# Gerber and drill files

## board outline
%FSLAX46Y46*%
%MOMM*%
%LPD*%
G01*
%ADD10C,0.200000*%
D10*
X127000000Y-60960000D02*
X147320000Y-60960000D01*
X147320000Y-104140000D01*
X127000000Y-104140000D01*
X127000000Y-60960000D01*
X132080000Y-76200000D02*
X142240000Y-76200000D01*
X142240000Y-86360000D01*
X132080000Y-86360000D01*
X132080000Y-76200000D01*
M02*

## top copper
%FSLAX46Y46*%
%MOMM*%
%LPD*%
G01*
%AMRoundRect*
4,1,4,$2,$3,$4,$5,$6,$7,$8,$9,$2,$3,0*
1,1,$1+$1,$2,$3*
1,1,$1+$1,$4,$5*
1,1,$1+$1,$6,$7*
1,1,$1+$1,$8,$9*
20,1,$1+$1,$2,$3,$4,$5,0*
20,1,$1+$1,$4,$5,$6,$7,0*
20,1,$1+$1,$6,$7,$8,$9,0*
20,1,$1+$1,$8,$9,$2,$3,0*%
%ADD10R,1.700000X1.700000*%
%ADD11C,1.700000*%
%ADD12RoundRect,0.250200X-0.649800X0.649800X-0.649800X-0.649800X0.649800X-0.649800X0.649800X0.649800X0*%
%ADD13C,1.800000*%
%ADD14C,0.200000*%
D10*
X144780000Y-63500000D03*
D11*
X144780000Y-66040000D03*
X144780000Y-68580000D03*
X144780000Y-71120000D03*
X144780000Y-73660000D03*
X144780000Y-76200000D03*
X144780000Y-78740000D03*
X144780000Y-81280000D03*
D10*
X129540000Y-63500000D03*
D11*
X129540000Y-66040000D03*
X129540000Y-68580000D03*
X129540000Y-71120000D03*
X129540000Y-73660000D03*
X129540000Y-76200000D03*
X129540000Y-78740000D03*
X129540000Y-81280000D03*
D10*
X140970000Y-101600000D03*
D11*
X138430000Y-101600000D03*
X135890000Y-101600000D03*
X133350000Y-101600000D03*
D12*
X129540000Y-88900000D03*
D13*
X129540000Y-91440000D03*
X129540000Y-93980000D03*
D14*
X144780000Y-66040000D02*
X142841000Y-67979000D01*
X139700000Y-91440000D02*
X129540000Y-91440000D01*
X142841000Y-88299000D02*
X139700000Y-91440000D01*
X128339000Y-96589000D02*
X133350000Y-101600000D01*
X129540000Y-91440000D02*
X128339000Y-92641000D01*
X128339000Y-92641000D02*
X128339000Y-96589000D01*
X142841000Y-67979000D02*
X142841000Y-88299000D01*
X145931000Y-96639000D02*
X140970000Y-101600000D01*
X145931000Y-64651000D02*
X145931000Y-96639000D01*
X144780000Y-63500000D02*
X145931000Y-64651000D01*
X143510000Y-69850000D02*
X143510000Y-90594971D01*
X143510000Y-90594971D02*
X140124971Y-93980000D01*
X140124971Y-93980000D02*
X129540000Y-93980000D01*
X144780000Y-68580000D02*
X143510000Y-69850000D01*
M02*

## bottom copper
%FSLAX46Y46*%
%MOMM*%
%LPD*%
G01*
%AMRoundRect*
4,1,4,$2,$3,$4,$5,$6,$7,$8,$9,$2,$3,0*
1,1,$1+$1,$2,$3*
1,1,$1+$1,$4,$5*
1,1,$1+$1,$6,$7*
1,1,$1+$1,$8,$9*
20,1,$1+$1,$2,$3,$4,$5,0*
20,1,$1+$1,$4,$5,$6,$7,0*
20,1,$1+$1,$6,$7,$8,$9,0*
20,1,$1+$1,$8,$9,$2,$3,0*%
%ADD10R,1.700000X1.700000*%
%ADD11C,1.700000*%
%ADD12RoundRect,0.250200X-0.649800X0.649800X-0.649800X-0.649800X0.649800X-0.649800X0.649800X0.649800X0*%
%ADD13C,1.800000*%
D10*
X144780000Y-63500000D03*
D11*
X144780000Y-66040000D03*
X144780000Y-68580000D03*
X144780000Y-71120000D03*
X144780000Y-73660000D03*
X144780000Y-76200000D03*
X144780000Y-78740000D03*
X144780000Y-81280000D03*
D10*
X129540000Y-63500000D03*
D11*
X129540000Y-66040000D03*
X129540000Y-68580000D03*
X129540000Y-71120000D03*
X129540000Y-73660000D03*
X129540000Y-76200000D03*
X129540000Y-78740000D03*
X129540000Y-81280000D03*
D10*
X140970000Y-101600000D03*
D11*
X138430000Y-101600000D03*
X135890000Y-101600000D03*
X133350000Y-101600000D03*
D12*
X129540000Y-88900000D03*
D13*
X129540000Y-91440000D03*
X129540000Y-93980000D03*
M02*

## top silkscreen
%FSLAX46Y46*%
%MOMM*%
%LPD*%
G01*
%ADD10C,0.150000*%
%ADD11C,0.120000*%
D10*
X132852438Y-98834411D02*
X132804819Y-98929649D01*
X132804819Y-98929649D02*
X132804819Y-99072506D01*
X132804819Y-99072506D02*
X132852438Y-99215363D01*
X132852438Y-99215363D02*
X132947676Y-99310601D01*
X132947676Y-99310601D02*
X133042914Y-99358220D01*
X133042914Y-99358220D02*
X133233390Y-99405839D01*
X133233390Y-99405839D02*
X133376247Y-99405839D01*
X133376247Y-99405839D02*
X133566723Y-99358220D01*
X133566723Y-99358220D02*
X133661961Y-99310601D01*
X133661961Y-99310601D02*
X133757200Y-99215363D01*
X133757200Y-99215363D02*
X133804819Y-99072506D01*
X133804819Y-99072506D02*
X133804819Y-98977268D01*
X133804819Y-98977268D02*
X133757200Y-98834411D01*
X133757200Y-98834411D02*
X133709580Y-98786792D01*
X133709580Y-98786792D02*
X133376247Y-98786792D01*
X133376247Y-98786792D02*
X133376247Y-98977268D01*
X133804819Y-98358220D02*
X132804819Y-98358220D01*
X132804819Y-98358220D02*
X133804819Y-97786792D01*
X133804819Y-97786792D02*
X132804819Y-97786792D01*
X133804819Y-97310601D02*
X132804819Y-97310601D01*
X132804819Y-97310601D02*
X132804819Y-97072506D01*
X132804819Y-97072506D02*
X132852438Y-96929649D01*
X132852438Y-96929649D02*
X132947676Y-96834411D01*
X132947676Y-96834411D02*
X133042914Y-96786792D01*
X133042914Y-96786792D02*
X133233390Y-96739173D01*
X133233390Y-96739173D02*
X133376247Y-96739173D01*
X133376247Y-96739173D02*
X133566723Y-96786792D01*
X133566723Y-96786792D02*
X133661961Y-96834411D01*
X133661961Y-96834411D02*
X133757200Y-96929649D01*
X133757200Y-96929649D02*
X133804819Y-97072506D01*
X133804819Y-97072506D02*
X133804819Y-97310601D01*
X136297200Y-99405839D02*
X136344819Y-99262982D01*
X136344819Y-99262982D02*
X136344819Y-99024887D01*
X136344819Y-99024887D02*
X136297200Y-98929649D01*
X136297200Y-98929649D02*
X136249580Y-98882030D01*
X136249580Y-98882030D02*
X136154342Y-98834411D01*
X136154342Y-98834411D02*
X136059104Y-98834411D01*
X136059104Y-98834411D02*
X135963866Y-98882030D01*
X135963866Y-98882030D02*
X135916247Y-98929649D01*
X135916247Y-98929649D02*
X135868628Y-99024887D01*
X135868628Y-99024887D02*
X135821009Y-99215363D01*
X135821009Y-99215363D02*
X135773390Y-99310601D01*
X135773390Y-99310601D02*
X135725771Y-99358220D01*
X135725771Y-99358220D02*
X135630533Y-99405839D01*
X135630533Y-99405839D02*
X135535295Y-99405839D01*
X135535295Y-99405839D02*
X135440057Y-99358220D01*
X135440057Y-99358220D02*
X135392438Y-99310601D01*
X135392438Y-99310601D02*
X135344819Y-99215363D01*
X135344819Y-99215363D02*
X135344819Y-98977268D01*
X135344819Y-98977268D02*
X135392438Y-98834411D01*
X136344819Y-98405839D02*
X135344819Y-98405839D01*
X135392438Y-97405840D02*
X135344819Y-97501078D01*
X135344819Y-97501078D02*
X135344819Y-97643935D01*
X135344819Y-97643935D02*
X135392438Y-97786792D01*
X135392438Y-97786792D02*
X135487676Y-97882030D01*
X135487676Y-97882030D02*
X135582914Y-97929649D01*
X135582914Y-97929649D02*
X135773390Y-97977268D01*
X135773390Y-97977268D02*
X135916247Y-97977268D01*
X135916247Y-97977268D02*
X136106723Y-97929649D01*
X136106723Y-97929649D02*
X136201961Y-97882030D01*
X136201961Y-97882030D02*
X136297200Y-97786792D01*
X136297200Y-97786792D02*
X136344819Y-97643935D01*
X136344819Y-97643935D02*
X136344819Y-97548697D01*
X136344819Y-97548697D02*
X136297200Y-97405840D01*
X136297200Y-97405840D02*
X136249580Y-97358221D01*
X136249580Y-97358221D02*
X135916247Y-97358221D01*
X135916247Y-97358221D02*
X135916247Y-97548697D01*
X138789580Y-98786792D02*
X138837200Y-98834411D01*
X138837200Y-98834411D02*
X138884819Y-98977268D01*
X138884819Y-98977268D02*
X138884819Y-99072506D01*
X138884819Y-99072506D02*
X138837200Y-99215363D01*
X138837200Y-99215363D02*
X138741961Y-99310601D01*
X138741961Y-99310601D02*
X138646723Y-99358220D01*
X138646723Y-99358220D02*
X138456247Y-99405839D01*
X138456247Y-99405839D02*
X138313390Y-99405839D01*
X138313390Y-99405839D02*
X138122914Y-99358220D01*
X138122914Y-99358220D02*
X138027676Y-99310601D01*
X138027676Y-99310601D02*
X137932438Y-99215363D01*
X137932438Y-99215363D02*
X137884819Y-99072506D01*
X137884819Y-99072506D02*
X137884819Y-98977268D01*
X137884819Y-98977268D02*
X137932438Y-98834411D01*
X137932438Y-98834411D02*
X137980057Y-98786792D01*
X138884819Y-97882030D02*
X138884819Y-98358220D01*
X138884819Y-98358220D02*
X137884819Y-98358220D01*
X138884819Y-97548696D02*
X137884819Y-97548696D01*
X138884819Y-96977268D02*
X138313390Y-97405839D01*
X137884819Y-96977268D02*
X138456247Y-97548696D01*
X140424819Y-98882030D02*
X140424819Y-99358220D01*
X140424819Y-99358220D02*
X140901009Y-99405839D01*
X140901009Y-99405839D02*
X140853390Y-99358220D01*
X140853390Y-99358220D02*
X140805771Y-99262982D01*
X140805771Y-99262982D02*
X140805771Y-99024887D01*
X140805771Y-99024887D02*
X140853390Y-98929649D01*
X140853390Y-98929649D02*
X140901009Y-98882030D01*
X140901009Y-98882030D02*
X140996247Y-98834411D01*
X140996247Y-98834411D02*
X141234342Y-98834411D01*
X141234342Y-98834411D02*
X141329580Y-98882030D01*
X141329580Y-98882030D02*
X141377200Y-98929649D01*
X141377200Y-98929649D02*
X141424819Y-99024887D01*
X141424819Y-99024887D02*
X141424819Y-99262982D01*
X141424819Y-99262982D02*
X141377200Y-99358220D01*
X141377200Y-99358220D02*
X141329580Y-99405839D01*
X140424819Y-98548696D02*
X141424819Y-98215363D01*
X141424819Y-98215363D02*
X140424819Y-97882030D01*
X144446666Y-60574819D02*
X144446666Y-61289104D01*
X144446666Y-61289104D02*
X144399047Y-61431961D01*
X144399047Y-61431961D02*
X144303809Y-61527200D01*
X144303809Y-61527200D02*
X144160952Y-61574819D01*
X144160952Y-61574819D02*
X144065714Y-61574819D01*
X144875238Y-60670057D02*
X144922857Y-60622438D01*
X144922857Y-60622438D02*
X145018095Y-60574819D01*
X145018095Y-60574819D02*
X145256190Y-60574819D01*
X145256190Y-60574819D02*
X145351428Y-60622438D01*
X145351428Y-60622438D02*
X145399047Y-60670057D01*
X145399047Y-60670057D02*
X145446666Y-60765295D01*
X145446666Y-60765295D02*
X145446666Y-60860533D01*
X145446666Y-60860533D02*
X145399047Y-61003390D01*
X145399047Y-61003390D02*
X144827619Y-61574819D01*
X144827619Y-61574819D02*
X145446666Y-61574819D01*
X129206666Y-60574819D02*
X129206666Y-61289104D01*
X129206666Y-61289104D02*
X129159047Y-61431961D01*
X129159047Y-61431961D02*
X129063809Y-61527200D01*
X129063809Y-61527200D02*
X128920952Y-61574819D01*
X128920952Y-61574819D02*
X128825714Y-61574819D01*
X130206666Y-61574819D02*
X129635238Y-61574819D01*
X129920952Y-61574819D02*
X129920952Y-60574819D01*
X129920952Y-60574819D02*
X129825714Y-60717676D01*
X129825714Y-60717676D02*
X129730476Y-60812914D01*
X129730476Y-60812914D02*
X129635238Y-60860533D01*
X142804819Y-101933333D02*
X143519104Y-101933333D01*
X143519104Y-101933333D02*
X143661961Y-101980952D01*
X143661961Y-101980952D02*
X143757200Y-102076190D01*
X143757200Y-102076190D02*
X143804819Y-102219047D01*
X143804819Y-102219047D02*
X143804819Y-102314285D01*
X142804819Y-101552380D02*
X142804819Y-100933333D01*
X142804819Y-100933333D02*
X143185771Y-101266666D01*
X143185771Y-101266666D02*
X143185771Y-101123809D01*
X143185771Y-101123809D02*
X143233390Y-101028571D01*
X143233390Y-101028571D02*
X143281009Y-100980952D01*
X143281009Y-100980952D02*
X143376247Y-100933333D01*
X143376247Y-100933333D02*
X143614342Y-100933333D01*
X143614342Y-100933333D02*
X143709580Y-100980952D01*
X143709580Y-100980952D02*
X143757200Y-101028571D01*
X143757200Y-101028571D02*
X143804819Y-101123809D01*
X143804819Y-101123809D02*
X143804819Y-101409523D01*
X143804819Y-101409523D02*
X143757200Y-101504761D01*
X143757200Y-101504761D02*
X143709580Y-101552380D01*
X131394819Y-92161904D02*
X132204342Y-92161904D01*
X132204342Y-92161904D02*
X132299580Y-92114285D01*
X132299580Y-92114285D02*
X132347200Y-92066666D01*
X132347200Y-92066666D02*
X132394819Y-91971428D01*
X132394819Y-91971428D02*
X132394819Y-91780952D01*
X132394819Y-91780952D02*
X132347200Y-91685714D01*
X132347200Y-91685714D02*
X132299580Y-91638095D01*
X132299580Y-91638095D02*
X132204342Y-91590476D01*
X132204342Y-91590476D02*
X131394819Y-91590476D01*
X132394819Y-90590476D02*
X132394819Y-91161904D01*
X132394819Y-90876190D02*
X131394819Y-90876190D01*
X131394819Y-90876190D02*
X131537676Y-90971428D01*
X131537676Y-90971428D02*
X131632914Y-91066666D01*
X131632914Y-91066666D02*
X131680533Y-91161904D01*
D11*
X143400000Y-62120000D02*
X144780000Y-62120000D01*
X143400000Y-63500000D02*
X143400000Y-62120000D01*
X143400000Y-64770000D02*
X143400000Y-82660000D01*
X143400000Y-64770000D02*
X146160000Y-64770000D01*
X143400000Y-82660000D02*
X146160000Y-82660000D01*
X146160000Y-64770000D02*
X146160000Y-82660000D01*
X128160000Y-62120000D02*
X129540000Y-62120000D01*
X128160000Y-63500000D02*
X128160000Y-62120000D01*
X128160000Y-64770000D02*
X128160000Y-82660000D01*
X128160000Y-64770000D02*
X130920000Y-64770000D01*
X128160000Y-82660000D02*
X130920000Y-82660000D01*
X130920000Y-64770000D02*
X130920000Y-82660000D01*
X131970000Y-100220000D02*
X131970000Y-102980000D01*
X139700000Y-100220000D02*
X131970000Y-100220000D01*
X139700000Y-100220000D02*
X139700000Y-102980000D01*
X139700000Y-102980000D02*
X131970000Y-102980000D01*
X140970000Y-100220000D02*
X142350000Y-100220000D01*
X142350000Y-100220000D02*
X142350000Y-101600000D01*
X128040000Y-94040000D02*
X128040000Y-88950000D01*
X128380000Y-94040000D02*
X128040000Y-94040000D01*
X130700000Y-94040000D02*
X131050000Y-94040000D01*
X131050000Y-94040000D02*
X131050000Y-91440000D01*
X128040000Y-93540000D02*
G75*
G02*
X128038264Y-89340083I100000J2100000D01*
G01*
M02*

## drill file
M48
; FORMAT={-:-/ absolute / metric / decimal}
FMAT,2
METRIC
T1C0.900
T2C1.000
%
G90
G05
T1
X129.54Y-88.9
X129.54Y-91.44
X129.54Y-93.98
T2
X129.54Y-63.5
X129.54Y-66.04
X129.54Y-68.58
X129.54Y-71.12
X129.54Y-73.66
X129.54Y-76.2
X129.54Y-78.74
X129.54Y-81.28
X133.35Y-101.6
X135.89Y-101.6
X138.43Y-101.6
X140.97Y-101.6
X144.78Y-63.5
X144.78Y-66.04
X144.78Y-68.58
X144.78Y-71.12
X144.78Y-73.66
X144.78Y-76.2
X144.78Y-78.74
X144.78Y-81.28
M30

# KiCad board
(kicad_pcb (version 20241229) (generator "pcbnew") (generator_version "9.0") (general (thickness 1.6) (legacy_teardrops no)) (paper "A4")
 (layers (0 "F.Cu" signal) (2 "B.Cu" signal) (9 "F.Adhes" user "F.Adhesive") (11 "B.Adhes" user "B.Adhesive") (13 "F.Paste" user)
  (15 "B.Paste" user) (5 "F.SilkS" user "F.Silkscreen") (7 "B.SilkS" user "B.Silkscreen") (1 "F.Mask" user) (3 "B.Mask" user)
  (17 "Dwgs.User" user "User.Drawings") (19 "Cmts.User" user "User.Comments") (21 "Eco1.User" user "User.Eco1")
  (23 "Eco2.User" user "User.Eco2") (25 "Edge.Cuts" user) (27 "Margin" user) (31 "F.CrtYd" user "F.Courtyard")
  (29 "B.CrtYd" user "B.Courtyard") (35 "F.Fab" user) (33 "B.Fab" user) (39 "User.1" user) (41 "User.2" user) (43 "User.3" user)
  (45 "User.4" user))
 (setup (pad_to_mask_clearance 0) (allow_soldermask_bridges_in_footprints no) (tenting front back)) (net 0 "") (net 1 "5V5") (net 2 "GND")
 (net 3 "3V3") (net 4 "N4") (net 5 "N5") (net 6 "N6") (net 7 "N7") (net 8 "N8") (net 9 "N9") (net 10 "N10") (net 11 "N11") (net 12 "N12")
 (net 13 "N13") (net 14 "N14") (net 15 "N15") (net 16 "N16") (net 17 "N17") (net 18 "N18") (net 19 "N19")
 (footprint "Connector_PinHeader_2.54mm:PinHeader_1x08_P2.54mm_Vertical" (layer "F.Cu") (at 144.78 63.5)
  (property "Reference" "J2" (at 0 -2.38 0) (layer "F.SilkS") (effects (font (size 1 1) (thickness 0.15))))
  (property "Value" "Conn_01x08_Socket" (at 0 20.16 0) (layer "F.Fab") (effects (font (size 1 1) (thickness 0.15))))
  (fp_line (start -1.38 -1.38) (end 0 -1.38) (stroke (width 0.12) (type solid)) (layer "F.SilkS"))
  (fp_line (start -1.38 0) (end -1.38 -1.38) (stroke (width 0.12) (type solid)) (layer "F.SilkS"))
  (fp_line (start -1.38 1.27) (end -1.38 19.16) (stroke (width 0.12) (type solid)) (layer "F.SilkS"))
  (fp_line (start -1.38 1.27) (end 1.38 1.27) (stroke (width 0.12) (type solid)) (layer "F.SilkS"))
  (fp_line (start -1.38 19.16) (end 1.38 19.16) (stroke (width 0.12) (type solid)) (layer "F.SilkS"))
  (fp_line (start 1.38 1.27) (end 1.38 19.16) (stroke (width 0.12) (type solid)) (layer "F.SilkS"))
  (pad "1" thru_hole rect (at 0 0) (size 1.7 1.7) (drill 1) (layers "*.Cu" "*.Mask") (remove_unused_layers no) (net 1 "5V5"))
  (pad "2" thru_hole circle (at 0 2.54) (size 1.7 1.7) (drill 1) (layers "*.Cu" "*.Mask") (remove_unused_layers no) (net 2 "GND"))
  (pad "3" thru_hole circle (at 0 5.08) (size 1.7 1.7) (drill 1) (layers "*.Cu" "*.Mask") (remove_unused_layers no) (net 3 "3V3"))
  (pad "4" thru_hole circle (at 0 7.62) (size 1.7 1.7) (drill 1) (layers "*.Cu" "*.Mask") (remove_unused_layers no) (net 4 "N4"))
  (pad "5" thru_hole circle (at 0 10.16) (size 1.7 1.7) (drill 1) (layers "*.Cu" "*.Mask") (remove_unused_layers no) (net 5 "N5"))
  (pad "6" thru_hole circle (at 0 12.7) (size 1.7 1.7) (drill 1) (layers "*.Cu" "*.Mask") (remove_unused_layers no) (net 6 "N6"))
  (pad "7" thru_hole circle (at 0 15.24) (size 1.7 1.7) (drill 1) (layers "*.Cu" "*.Mask") (remove_unused_layers no) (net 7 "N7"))
  (pad "8" thru_hole circle (at 0 17.78) (size 1.7 1.7) (drill 1) (layers "*.Cu" "*.Mask") (remove_unused_layers no) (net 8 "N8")))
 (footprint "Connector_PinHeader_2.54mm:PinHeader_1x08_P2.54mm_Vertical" (layer "F.Cu") (at 129.54 63.5)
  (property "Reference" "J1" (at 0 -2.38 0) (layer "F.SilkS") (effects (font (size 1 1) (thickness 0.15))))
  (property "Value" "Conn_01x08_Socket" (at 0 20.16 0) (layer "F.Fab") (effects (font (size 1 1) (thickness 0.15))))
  (fp_line (start -1.38 -1.38) (end 0 -1.38) (stroke (width 0.12) (type solid)) (layer "F.SilkS"))
  (fp_line (start -1.38 0) (end -1.38 -1.38) (stroke (width 0.12) (type solid)) (layer "F.SilkS"))
  (fp_line (start -1.38 1.27) (end -1.38 19.16) (stroke (width 0.12) (type solid)) (layer "F.SilkS"))
  (fp_line (start -1.38 1.27) (end 1.38 1.27) (stroke (width 0.12) (type solid)) (layer "F.SilkS"))
  (fp_line (start -1.38 19.16) (end 1.38 19.16) (stroke (width 0.12) (type solid)) (layer "F.SilkS"))
  (fp_line (start 1.38 1.27) (end 1.38 19.16) (stroke (width 0.12) (type solid)) (layer "F.SilkS"))
  (pad "1" thru_hole rect (at 0 0) (size 1.7 1.7) (drill 1) (layers "*.Cu" "*.Mask") (remove_unused_layers no) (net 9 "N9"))
  (pad "2" thru_hole circle (at 0 2.54) (size 1.7 1.7) (drill 1) (layers "*.Cu" "*.Mask") (remove_unused_layers no) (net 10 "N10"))
  (pad "3" thru_hole circle (at 0 5.08) (size 1.7 1.7) (drill 1) (layers "*.Cu" "*.Mask") (remove_unused_layers no) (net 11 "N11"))
  (pad "4" thru_hole circle (at 0 7.62) (size 1.7 1.7) (drill 1) (layers "*.Cu" "*.Mask") (remove_unused_layers no) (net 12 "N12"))
  (pad "5" thru_hole circle (at 0 10.16) (size 1.7 1.7) (drill 1) (layers "*.Cu" "*.Mask") (remove_unused_layers no) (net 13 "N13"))
  (pad "6" thru_hole circle (at 0 12.7) (size 1.7 1.7) (drill 1) (layers "*.Cu" "*.Mask") (remove_unused_layers no) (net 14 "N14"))
  (pad "7" thru_hole circle (at 0 15.24) (size 1.7 1.7) (drill 1) (layers "*.Cu" "*.Mask") (remove_unused_layers no) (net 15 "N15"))
  (pad "8" thru_hole circle (at 0 17.78) (size 1.7 1.7) (drill 1) (layers "*.Cu" "*.Mask") (remove_unused_layers no) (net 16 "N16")))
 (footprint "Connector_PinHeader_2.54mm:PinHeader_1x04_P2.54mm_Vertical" (layer "F.Cu") (at 140.97 101.6 -90)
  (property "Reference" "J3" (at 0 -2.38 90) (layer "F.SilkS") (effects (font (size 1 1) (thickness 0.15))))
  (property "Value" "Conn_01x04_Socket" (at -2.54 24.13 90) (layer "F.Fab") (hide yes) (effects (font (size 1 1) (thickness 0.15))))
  (fp_line (start -1.38 9) (end 1.38 9) (stroke (width 0.12) (type solid)) (layer "F.SilkS"))
  (fp_line (start -1.38 1.27) (end -1.38 9) (stroke (width 0.12) (type solid)) (layer "F.SilkS"))
  (fp_line (start -1.38 1.27) (end 1.38 1.27) (stroke (width 0.12) (type solid)) (layer "F.SilkS"))
  (fp_line (start 1.38 1.27) (end 1.38 9) (stroke (width 0.12) (type solid)) (layer "F.SilkS"))
  (fp_line (start -1.38 0) (end -1.38 -1.38) (stroke (width 0.12) (type solid)) (layer "F.SilkS"))
  (fp_line (start -1.38 -1.38) (end 0 -1.38) (stroke (width 0.12) (type solid)) (layer "F.SilkS"))
  (pad "1" thru_hole rect (at 0 0 270) (size 1.7 1.7) (drill 1) (layers "*.Cu" "*.Mask") (remove_unused_layers no) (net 1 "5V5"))
  (pad "2" thru_hole circle (at 0 2.54 270) (size 1.7 1.7) (drill 1) (layers "*.Cu" "*.Mask") (remove_unused_layers no) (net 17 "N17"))
  (pad "3" thru_hole circle (at 0 5.08 270) (size 1.7 1.7) (drill 1) (layers "*.Cu" "*.Mask") (remove_unused_layers no) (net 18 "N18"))
  (pad "4" thru_hole circle (at 0 7.62 270) (size 1.7 1.7) (drill 1) (layers "*.Cu" "*.Mask") (remove_unused_layers no) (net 2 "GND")))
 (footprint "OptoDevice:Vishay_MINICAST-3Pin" (layer "F.Cu") (at 129.54 88.9 -90)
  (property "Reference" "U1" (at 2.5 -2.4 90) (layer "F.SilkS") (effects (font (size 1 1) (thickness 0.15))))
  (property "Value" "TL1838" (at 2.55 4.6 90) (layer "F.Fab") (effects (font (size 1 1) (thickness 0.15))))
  (fp_line (start 5.14 1.5) (end 0.05 1.5) (stroke (width 0.12) (type solid)) (layer "F.SilkS"))
  (fp_line (start 5.14 1.16) (end 5.14 1.5) (stroke (width 0.12) (type solid)) (layer "F.SilkS"))
  (fp_line (start 5.14 -1.16) (end 5.14 -1.51) (stroke (width 0.12) (type solid)) (layer "F.SilkS"))
  (fp_line (start 5.14 -1.51) (end 2.54 -1.51) (stroke (width 0.12) (type solid)) (layer "F.SilkS"))
  (fp_arc (start 4.64 1.5) (mid 2.540869 3.502379) (end 0.440083 1.501736) (stroke (width 0.12) (type solid)) (layer "F.SilkS"))
  (pad "1" thru_hole roundrect (at 0 0 270) (size 1.8 1.8) (drill 0.9) (layers "*.Cu" "*.Mask") (remove_unused_layers no)
   (roundrect_rratio 0.139) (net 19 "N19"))
  (pad "2" thru_hole circle (at 2.54 0 270) (size 1.8 1.8) (drill 0.9) (layers "*.Cu" "*.Mask") (remove_unused_layers no) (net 2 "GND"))
  (pad "3" thru_hole circle (at 5.08 0 270) (size 1.8 1.8) (drill 0.9) (layers "*.Cu" "*.Mask") (remove_unused_layers no) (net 3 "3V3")))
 (gr_rect (start 127 60.96) (end 147.32 104.14) (stroke (width 0.2) (type solid)) (fill no) (layer "Edge.Cuts"))
 (gr_rect (start 132.08 76.2) (end 142.24 86.36) (stroke (width 0.2) (type solid)) (fill no) (layer "Edge.Cuts"))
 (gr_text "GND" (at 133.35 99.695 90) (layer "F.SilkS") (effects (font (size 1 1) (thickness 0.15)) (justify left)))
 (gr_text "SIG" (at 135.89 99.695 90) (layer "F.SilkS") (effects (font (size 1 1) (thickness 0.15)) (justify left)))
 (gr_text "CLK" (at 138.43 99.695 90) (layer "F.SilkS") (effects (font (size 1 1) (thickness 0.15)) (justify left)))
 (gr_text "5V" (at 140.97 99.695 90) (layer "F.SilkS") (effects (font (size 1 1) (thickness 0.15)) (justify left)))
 (segment (start 144.78 66.04) (end 142.841 67.979) (width 0.2) (layer "F.Cu") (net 2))
 (segment (start 139.7 91.44) (end 129.54 91.44) (width 0.2) (layer "F.Cu") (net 2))
 (segment (start 142.841 88.299) (end 139.7 91.44) (width 0.2) (layer "F.Cu") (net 2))
 (segment (start 128.339 96.589) (end 133.35 101.6) (width 0.2) (layer "F.Cu") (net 2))
 (segment (start 129.54 91.44) (end 128.339 92.641) (width 0.2) (layer "F.Cu") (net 2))
 (segment (start 128.339 92.641) (end 128.339 96.589) (width 0.2) (layer "F.Cu") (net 2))
 (segment (start 142.841 67.979) (end 142.841 88.299) (width 0.2) (layer "F.Cu") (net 2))
 (segment (start 145.931 96.639) (end 140.97 101.6) (width 0.2) (layer "F.Cu") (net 1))
 (segment (start 145.931 64.651) (end 145.931 96.639) (width 0.2) (layer "F.Cu") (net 1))
 (segment (start 144.78 63.5) (end 145.931 64.651) (width 0.2) (layer "F.Cu") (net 1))
 (segment (start 143.51 69.85) (end 143.51 90.594971) (width 0.2) (layer "F.Cu") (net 3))
 (segment (start 143.51 90.594971) (end 140.124971 93.98) (width 0.2) (layer "F.Cu") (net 3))
 (segment (start 140.124971 93.98) (end 129.54 93.98) (width 0.2) (layer "F.Cu") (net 3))
 (segment (start 144.78 68.58) (end 143.51 69.85) (width 0.2) (layer "F.Cu") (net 3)))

